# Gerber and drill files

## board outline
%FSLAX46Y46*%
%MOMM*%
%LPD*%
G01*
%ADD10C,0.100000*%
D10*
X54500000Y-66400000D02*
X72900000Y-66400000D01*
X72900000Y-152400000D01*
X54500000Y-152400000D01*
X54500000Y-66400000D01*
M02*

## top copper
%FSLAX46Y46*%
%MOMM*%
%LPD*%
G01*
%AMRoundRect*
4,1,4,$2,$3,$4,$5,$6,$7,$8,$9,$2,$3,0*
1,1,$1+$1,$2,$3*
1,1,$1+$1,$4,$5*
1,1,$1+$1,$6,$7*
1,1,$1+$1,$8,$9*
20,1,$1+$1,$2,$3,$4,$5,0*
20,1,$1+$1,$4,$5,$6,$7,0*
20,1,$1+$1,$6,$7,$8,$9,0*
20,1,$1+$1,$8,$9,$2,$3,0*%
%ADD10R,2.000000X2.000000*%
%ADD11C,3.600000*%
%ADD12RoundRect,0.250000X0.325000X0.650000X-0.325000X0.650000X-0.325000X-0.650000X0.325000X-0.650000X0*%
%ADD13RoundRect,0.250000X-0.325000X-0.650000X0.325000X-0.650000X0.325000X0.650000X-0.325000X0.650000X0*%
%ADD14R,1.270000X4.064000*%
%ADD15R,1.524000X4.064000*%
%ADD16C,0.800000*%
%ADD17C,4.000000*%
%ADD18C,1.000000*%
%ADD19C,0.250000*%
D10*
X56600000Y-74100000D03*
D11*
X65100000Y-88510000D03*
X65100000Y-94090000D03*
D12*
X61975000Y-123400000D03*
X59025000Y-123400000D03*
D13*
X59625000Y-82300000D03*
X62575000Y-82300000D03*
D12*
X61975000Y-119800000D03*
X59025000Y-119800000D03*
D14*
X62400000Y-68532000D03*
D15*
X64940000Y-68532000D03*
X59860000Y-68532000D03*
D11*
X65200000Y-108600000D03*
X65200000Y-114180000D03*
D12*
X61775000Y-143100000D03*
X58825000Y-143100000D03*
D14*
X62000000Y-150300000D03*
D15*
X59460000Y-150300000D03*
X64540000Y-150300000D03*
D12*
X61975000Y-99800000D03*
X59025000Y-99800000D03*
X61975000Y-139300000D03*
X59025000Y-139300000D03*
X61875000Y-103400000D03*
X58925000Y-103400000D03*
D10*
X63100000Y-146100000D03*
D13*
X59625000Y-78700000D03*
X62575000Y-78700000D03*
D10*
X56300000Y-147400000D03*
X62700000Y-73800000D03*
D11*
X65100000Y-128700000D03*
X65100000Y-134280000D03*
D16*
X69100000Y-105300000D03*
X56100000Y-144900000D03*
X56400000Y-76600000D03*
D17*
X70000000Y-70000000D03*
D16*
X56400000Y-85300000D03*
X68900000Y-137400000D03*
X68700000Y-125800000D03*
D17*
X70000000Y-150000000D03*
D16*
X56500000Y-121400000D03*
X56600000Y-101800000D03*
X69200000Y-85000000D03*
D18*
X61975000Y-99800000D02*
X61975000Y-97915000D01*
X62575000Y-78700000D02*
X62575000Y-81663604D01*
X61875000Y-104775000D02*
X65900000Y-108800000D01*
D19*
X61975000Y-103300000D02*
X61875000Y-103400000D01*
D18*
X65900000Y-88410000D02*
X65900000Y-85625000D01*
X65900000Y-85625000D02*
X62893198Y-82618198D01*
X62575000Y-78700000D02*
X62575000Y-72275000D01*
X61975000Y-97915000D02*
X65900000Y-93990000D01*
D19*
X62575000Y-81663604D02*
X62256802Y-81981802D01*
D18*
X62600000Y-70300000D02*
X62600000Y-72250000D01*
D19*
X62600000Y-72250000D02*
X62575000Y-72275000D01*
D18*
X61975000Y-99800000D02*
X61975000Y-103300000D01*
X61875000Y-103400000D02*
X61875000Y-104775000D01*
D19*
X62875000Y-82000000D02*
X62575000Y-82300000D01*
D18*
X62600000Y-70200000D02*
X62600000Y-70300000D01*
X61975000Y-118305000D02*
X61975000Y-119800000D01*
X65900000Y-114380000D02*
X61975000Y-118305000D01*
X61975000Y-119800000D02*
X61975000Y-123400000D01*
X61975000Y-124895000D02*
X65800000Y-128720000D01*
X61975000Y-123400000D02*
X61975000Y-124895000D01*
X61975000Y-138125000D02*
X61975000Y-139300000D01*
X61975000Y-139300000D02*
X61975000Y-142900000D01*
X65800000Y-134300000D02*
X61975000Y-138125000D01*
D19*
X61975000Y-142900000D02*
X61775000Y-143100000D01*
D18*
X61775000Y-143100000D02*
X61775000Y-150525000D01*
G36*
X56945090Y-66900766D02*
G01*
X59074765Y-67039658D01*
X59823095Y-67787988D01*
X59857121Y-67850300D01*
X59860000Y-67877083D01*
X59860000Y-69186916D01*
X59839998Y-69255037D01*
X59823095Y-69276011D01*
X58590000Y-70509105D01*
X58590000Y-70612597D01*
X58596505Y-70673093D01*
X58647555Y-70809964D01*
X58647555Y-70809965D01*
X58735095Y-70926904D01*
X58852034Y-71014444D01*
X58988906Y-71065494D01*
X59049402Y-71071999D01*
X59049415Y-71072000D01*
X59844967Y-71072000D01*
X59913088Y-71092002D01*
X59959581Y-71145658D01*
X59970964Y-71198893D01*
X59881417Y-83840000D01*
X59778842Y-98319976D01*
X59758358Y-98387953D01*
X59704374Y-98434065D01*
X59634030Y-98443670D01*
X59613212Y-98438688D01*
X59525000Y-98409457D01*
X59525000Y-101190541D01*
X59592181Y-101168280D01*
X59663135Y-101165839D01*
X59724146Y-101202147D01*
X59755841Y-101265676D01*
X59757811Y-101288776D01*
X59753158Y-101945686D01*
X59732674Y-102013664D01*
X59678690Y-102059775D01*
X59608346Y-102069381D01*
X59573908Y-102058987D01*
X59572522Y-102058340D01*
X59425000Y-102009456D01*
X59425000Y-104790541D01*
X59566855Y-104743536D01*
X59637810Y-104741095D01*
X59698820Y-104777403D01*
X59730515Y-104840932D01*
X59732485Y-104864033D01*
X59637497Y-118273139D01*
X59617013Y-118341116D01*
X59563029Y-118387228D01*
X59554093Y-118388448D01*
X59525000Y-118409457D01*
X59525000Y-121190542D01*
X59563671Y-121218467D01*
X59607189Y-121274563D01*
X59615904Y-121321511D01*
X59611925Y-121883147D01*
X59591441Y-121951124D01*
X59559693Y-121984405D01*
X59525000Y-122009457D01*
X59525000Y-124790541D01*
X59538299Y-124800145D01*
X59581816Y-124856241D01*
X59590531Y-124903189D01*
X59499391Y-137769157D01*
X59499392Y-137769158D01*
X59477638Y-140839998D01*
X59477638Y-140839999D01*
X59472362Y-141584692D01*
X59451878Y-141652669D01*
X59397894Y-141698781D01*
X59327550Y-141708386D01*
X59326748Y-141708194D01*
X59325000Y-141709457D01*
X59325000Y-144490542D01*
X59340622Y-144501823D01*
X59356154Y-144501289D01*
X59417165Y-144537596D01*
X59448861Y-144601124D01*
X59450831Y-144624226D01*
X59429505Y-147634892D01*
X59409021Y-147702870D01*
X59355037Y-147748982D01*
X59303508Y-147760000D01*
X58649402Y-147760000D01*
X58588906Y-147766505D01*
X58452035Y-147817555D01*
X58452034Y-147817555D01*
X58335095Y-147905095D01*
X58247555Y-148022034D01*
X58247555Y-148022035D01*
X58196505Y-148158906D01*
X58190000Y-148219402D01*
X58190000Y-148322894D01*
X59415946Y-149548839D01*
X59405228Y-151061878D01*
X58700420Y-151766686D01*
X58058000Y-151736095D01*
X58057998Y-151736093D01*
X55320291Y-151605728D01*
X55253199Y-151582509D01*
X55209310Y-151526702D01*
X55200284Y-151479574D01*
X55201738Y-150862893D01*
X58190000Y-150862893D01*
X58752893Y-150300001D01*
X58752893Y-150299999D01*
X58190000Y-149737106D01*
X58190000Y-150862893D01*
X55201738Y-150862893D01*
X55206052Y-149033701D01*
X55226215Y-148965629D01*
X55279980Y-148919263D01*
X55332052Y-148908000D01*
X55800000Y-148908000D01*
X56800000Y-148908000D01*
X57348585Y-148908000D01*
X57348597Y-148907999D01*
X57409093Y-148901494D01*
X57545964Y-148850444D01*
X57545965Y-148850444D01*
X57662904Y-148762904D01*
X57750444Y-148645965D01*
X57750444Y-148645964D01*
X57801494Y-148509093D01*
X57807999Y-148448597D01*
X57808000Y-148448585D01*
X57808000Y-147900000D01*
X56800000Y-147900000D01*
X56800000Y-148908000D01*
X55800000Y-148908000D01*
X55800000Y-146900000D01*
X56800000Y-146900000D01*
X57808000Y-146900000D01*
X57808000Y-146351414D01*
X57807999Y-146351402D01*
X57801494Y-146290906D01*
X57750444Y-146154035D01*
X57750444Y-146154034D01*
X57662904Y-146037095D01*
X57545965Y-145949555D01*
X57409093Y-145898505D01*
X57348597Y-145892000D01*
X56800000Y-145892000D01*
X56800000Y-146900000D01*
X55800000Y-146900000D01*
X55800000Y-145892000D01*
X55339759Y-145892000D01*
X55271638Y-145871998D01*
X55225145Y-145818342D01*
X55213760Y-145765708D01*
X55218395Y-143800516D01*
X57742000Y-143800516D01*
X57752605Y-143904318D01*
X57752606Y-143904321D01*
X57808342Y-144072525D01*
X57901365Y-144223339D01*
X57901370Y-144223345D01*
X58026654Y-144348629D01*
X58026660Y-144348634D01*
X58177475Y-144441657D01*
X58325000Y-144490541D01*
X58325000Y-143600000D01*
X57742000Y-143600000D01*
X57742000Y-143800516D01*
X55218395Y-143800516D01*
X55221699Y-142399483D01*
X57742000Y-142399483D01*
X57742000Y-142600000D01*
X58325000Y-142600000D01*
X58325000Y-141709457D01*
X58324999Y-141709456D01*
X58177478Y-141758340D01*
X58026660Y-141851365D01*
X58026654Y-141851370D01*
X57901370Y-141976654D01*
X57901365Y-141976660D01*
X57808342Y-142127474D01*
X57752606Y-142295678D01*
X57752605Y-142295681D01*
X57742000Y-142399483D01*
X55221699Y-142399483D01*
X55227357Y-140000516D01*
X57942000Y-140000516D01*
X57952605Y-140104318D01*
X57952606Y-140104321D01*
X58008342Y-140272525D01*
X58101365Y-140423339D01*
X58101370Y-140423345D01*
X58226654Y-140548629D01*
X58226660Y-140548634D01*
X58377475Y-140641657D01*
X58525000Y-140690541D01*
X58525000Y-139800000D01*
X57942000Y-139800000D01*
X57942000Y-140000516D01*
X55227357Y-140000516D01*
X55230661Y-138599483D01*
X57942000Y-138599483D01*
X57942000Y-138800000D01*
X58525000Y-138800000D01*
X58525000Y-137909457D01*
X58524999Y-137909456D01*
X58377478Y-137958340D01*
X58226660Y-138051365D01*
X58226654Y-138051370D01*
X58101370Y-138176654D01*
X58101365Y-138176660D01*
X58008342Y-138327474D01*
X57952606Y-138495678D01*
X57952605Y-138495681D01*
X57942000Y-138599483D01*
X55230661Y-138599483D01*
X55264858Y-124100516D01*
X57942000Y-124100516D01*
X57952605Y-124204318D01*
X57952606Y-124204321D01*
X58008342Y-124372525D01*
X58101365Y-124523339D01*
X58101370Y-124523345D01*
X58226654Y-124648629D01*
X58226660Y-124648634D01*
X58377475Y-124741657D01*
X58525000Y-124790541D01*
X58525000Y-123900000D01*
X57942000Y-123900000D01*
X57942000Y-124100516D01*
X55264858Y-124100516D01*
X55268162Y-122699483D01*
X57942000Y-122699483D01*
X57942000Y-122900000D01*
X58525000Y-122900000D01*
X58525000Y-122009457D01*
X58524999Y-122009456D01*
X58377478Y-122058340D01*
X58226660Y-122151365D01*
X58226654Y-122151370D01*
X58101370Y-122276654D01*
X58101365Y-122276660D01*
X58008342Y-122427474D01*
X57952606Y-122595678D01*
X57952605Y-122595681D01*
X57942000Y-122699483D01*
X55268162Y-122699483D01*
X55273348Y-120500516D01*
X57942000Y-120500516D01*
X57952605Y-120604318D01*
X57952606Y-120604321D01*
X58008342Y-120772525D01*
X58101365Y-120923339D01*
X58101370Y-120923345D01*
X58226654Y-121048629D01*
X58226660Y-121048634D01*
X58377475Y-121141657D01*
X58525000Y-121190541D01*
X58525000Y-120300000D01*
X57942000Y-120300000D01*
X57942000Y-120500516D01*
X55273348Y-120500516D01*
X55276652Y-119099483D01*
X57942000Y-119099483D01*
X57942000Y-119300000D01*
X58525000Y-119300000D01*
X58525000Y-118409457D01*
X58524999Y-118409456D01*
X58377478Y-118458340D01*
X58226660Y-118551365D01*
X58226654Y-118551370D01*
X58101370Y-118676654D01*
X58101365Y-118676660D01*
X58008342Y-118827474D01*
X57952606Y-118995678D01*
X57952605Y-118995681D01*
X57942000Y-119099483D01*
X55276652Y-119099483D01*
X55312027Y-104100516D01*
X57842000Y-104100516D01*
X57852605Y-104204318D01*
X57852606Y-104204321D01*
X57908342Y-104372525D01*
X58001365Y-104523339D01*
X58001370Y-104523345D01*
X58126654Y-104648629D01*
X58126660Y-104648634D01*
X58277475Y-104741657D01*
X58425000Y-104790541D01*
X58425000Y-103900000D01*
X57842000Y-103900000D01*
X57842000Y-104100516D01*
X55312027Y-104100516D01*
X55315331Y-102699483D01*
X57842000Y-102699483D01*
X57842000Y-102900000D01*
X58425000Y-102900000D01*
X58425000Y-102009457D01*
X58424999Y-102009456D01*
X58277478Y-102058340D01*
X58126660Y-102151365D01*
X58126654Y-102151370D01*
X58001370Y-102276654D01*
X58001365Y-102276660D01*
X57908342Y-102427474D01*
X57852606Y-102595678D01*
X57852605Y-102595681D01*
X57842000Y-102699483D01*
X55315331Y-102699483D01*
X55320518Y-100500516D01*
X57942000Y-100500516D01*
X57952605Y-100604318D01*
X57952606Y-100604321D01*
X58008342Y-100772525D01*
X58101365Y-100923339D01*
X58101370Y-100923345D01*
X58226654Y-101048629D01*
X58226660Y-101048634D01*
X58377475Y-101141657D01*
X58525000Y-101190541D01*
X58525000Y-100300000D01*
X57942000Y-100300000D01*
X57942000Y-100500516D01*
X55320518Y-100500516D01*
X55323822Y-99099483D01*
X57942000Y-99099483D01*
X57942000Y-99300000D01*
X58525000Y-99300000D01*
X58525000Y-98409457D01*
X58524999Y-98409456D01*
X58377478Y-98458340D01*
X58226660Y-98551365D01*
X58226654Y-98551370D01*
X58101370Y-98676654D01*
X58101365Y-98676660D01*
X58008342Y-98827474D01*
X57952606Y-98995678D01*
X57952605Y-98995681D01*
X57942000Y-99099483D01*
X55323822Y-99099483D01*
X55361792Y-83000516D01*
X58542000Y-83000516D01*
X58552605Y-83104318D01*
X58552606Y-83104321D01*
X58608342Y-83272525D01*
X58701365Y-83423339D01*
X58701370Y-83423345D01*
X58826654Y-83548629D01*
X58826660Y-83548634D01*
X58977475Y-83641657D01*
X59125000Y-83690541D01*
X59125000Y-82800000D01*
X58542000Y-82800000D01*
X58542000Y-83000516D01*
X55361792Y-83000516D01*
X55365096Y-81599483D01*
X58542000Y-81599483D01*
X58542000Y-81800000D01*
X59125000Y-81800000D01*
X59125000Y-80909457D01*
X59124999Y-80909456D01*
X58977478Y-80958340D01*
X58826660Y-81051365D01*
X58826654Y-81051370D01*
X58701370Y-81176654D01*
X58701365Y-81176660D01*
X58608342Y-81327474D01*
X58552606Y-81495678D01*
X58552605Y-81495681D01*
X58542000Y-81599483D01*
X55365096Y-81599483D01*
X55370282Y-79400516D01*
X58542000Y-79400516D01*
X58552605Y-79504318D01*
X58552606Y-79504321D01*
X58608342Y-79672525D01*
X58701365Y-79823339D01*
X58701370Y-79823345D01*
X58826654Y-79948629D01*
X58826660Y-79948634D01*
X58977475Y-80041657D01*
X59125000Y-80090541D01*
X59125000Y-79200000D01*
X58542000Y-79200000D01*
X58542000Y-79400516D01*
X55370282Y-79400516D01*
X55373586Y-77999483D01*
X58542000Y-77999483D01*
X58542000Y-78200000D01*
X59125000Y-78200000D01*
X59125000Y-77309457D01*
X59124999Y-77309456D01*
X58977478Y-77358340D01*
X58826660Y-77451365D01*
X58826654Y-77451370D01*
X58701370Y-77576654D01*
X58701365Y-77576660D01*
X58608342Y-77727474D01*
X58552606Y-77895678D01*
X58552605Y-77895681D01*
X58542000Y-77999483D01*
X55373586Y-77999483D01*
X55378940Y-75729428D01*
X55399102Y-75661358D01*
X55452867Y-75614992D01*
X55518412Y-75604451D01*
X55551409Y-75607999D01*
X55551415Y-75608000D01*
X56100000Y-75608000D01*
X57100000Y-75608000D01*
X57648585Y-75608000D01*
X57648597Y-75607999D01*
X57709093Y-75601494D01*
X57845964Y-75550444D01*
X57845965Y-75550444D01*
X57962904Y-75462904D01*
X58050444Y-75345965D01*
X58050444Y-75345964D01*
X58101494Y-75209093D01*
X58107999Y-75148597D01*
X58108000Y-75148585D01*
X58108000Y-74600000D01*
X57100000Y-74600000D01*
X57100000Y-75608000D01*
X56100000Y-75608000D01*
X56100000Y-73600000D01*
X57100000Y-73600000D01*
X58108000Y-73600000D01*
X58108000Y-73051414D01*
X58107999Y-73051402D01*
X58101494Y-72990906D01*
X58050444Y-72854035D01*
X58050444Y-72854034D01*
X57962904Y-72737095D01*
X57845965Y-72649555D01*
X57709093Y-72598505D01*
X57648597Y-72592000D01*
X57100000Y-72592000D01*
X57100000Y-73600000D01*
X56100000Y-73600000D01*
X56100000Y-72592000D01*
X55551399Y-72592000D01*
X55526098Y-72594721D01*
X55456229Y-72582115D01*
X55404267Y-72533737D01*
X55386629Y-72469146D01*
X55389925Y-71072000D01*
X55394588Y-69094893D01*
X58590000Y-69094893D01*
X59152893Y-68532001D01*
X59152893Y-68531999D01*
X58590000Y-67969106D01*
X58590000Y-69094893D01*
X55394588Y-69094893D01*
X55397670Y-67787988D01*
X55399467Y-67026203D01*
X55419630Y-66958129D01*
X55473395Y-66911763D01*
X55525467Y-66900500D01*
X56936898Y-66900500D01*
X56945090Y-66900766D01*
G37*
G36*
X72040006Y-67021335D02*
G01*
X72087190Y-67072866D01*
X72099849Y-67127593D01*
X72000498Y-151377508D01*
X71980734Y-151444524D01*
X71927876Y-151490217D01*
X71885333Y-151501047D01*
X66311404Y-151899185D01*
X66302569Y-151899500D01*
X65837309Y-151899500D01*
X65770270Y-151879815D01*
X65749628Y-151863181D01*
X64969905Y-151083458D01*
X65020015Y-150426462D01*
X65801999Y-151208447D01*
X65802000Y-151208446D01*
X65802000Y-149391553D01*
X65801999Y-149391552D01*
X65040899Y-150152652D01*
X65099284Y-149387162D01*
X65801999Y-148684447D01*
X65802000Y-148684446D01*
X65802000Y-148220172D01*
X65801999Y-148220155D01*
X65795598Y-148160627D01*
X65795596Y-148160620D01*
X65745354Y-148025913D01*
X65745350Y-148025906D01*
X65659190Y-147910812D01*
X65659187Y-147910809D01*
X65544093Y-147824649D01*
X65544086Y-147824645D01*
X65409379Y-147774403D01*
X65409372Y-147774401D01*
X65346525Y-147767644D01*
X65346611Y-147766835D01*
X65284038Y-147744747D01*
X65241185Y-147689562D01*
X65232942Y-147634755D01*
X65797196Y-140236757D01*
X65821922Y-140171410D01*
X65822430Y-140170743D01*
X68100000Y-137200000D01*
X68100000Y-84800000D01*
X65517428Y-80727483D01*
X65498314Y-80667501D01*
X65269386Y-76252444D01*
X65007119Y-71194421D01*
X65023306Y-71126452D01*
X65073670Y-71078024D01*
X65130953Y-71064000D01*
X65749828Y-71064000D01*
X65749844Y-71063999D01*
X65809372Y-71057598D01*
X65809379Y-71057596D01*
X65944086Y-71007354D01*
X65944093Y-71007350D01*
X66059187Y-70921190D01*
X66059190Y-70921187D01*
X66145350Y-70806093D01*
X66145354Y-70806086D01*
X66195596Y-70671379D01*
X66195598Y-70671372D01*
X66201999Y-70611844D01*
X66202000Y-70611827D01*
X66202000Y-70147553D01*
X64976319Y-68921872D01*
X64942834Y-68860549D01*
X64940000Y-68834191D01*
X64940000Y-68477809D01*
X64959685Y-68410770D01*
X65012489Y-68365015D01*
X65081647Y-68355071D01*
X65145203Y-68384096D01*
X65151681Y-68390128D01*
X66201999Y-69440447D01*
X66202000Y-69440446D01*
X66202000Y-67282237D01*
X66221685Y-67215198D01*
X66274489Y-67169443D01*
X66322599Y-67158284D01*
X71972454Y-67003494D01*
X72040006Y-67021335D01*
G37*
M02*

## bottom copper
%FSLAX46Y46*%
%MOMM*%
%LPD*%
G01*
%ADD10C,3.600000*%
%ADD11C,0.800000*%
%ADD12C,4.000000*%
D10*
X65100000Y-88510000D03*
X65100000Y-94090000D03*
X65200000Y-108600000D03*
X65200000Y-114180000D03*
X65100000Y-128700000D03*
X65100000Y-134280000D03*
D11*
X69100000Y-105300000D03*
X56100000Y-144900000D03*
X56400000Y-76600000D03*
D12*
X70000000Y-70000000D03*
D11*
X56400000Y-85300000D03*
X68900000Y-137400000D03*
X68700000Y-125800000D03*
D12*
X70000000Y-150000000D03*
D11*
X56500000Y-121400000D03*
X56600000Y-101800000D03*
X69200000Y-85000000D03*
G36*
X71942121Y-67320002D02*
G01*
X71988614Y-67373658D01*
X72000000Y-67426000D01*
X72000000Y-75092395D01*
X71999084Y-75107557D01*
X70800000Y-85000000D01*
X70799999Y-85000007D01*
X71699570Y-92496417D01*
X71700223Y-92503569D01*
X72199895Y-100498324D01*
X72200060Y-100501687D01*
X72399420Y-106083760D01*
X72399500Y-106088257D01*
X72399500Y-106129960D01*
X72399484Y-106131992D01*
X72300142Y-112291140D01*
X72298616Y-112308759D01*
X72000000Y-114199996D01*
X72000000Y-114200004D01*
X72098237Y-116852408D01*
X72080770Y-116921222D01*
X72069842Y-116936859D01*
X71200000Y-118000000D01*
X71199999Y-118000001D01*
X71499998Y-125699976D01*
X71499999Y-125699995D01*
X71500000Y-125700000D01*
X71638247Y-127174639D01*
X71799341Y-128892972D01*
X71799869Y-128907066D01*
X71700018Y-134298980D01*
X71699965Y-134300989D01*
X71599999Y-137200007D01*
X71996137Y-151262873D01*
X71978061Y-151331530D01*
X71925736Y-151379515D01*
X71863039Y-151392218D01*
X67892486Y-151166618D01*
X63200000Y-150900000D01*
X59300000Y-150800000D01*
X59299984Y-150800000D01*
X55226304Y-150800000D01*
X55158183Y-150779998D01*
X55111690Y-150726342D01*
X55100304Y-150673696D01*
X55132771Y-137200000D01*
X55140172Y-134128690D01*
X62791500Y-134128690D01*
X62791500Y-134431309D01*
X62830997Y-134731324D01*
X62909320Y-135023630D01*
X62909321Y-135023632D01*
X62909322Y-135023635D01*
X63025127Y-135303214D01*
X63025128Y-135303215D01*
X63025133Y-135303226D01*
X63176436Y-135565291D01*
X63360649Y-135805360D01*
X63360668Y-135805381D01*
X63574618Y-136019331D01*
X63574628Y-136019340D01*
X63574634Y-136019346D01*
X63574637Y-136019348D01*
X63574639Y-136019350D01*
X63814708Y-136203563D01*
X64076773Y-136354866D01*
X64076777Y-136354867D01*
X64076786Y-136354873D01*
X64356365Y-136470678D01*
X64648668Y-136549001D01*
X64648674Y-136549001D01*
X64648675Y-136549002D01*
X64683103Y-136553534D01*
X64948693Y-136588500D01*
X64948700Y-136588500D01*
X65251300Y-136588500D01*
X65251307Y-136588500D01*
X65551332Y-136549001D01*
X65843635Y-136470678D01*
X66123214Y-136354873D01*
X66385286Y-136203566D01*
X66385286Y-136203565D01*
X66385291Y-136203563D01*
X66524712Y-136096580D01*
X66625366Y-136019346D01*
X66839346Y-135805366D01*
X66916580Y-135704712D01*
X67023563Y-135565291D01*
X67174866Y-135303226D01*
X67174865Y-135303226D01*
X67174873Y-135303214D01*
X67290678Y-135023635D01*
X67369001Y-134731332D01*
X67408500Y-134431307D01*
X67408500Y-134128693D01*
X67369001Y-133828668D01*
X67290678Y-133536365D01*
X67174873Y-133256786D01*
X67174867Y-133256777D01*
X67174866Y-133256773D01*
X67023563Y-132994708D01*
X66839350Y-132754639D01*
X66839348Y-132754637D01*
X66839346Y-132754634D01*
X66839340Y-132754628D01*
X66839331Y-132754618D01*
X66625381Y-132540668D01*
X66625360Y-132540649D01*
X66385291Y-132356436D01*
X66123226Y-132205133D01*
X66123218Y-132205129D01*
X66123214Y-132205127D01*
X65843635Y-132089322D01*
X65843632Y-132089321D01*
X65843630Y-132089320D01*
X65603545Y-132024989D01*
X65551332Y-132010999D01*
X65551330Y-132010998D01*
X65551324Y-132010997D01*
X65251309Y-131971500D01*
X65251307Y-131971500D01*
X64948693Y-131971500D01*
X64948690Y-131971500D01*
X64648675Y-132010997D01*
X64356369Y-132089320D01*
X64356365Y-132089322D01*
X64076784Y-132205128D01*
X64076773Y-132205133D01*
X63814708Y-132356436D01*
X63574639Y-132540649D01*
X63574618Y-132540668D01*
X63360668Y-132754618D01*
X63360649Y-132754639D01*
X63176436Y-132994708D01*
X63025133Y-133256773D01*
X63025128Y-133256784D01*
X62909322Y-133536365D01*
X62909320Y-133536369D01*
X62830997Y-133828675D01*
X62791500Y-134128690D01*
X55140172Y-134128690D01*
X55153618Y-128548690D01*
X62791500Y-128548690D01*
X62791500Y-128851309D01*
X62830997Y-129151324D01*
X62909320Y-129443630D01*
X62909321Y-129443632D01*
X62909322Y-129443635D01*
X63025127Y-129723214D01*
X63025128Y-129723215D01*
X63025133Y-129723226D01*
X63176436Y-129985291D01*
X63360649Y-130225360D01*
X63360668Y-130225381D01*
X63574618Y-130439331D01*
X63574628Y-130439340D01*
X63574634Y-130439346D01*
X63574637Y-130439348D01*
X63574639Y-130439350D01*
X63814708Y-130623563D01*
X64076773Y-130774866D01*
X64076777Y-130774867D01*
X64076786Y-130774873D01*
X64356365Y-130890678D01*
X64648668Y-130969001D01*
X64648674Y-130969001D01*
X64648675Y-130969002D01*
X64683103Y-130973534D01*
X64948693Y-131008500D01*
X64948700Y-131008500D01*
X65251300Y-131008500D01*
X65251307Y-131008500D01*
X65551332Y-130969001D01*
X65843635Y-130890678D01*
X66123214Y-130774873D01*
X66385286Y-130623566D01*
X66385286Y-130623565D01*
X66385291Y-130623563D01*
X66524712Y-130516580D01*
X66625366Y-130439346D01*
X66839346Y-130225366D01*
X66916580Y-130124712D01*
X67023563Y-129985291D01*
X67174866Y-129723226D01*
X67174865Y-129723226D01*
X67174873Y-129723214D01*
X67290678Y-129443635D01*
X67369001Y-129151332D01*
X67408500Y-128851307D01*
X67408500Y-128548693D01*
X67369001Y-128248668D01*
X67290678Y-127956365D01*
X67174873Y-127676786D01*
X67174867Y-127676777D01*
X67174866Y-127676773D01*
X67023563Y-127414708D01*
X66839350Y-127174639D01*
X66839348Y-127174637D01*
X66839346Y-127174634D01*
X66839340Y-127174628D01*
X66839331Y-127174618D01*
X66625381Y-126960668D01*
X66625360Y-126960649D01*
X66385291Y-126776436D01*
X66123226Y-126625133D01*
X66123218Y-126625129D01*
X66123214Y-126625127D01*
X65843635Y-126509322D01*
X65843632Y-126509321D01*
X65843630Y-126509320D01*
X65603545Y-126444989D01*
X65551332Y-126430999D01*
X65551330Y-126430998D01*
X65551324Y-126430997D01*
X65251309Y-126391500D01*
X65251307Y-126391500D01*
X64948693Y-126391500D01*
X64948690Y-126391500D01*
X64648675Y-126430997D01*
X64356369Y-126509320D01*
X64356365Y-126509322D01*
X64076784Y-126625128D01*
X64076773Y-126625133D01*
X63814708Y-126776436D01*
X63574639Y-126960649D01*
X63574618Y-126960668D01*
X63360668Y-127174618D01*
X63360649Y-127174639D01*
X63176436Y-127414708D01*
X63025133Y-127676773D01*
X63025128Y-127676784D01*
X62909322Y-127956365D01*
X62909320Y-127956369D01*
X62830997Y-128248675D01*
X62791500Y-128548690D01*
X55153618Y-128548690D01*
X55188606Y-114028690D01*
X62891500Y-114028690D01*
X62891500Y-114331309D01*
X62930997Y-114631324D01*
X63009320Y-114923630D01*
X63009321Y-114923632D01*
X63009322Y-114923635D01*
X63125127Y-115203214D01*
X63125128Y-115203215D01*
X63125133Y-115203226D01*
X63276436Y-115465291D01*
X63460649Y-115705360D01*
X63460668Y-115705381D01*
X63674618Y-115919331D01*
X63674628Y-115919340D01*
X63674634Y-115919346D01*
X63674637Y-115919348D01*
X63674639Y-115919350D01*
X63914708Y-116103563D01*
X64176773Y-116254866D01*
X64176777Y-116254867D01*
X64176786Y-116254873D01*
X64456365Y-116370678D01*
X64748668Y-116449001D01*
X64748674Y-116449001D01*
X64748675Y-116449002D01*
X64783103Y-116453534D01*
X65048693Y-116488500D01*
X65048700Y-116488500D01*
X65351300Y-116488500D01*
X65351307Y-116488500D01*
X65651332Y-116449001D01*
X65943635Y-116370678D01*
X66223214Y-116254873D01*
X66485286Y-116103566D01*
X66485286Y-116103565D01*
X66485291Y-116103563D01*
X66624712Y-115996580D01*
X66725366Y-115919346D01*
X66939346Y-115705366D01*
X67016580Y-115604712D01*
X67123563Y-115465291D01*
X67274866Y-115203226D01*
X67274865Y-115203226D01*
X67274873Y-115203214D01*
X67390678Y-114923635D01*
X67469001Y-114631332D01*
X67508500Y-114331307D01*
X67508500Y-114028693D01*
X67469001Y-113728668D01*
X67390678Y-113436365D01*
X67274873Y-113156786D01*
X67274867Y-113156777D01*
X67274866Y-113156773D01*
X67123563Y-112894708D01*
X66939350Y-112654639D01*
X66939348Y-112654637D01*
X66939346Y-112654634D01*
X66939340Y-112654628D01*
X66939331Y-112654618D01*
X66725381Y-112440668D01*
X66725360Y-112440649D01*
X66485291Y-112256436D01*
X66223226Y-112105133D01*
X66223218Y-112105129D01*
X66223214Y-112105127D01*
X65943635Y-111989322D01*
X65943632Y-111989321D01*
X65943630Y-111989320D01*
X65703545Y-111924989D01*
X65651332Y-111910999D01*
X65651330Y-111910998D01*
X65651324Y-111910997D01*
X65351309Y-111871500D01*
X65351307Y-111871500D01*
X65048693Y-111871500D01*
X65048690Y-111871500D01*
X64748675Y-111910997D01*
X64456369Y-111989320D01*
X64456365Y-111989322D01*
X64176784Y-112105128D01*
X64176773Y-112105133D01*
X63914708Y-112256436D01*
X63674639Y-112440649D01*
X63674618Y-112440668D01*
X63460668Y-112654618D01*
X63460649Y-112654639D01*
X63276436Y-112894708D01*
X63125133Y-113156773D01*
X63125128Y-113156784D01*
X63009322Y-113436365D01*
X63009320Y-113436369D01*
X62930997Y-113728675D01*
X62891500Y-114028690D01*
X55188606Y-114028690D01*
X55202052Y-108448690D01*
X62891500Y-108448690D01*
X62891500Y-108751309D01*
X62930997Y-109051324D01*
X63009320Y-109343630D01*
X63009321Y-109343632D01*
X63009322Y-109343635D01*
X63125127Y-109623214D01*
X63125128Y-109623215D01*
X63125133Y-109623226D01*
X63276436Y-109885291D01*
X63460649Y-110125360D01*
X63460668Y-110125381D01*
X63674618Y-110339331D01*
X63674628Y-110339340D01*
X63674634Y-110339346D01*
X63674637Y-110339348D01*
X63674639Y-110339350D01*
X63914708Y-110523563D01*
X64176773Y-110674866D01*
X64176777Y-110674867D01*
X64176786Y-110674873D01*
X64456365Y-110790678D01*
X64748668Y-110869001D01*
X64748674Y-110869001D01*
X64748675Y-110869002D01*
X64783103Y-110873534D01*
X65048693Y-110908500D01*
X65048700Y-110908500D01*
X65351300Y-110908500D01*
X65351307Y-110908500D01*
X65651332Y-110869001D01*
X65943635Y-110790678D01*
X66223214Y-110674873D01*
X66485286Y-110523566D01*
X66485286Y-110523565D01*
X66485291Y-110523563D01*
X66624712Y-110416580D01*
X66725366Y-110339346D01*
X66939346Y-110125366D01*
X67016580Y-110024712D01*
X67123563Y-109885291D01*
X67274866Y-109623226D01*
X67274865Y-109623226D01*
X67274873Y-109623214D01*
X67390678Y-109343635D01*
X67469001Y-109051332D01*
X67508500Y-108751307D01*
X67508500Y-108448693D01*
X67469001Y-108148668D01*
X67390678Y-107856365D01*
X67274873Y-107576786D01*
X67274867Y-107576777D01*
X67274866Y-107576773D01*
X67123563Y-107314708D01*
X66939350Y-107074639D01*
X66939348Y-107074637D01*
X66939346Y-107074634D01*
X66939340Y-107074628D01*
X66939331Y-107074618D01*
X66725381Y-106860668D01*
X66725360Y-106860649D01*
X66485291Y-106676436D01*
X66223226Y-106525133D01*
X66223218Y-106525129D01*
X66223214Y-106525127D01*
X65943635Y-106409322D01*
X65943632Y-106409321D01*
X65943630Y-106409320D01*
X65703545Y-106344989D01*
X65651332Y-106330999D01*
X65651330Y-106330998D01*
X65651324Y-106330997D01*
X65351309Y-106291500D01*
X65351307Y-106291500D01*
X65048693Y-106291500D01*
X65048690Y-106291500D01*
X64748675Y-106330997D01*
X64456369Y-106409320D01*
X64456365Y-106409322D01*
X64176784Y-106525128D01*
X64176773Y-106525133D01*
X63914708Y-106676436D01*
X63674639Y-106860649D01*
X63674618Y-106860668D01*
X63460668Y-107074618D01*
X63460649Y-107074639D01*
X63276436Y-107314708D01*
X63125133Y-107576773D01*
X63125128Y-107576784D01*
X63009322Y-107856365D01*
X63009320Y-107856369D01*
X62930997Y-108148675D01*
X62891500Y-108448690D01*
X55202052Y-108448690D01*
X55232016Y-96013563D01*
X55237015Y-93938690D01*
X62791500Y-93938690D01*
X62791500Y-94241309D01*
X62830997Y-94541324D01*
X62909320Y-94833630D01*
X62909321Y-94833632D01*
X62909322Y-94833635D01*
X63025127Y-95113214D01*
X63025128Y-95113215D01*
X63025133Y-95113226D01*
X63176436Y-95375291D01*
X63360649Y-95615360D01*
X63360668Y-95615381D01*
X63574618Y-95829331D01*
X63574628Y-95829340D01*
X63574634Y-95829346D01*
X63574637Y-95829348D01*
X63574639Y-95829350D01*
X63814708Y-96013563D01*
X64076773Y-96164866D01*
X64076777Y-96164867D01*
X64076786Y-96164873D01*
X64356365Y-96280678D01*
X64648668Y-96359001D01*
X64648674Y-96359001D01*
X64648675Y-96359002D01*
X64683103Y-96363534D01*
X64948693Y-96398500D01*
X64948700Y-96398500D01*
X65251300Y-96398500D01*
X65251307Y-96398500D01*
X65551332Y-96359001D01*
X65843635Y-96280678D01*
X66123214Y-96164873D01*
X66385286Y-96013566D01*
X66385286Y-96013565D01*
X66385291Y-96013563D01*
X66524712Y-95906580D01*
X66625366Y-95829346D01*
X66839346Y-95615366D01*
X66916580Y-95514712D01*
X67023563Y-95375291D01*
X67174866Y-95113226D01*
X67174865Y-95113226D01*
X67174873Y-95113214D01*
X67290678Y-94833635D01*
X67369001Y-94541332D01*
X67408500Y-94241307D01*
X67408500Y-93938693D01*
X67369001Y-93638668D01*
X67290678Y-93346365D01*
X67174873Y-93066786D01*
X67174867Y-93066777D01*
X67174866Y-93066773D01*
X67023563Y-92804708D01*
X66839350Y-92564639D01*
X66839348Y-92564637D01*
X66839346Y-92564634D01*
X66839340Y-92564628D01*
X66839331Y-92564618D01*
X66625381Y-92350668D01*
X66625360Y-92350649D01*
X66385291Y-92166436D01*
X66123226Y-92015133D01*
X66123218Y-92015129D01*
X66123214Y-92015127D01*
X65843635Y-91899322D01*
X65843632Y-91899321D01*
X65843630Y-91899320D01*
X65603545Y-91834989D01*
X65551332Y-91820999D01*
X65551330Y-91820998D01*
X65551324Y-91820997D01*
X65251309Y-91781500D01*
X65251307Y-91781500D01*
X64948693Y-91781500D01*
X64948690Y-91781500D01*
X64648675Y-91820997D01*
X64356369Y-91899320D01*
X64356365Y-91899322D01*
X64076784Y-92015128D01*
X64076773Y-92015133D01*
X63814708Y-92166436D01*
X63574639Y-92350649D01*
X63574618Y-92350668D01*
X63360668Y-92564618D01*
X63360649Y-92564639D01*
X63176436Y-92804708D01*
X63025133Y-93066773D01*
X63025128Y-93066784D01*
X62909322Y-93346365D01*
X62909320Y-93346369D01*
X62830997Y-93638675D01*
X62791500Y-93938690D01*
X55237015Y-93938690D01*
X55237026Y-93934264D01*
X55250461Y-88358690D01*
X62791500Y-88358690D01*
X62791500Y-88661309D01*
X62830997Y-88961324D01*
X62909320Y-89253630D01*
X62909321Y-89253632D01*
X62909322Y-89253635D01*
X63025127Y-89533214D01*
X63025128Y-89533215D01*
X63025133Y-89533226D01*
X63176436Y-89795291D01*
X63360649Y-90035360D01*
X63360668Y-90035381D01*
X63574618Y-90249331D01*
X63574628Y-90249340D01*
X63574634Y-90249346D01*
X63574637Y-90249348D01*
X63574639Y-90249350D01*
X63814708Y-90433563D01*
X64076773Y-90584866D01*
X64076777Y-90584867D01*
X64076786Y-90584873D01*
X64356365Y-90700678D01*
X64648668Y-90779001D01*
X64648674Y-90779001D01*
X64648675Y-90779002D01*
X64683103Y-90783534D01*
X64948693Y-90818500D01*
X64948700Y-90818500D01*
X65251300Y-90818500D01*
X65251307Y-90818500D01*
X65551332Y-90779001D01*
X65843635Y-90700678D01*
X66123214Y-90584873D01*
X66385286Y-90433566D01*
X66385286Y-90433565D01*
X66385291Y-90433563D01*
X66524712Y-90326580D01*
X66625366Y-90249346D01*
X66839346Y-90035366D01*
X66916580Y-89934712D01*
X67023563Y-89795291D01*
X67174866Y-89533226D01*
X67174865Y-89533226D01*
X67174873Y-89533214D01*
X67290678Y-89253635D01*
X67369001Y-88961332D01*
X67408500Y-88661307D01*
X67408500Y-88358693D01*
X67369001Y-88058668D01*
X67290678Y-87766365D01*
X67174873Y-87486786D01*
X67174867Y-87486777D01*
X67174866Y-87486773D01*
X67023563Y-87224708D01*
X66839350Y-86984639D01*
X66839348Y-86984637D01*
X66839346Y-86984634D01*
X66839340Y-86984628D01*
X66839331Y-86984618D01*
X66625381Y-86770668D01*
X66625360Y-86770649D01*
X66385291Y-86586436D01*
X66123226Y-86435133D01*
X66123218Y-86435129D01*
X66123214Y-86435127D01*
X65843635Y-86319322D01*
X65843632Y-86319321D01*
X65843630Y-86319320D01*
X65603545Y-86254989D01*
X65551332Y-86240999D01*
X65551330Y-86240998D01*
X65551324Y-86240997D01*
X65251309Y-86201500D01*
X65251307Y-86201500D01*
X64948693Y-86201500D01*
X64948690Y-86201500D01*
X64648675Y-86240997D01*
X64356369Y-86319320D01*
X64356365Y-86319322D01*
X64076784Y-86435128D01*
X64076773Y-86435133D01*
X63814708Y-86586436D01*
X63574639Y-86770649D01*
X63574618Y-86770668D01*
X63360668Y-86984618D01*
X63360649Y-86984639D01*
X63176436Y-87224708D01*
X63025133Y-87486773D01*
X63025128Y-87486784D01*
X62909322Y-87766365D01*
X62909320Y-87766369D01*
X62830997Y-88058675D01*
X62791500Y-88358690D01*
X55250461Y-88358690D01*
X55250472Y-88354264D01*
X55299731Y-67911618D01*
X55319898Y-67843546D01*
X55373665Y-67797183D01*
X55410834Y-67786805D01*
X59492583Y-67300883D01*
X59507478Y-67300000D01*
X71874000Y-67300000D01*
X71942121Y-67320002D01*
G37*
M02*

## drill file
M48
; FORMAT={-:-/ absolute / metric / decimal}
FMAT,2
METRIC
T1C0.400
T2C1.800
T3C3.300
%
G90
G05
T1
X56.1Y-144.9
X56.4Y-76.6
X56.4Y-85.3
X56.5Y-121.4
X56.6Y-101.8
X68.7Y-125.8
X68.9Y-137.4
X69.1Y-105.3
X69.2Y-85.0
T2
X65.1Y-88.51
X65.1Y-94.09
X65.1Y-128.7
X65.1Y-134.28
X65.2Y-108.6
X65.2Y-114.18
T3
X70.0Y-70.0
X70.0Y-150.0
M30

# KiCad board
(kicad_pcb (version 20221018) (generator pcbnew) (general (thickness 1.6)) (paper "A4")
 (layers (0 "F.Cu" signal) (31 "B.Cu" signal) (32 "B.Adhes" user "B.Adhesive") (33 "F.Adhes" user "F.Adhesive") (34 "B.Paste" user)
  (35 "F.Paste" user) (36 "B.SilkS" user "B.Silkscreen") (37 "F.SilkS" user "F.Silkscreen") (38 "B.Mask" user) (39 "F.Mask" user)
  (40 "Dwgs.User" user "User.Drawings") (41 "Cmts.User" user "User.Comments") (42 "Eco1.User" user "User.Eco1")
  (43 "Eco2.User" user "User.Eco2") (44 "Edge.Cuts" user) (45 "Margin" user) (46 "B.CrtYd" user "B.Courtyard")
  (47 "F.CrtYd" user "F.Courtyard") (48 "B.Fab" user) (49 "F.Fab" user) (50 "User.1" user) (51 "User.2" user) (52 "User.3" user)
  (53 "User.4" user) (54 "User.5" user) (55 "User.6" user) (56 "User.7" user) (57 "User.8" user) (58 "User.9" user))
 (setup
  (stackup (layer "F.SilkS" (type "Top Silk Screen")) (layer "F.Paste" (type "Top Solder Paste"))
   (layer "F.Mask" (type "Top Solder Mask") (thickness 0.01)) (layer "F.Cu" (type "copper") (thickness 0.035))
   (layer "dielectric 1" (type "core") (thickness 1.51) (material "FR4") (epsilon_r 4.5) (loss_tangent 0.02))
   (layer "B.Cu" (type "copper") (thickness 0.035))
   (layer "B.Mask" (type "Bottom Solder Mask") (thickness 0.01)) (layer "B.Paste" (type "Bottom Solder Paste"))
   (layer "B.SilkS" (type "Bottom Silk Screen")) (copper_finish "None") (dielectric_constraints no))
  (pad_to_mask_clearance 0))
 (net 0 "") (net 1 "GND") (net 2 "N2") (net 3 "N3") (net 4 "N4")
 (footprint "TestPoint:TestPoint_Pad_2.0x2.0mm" (layer "F.Cu") (at 56.6 74.1)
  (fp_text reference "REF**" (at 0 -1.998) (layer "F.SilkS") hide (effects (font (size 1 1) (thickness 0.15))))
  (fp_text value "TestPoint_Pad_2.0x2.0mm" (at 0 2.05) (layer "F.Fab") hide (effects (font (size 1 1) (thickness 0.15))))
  (pad "1" smd rect (at 0 0) (size 2 2) (layers "F.Cu" "F.Mask") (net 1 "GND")))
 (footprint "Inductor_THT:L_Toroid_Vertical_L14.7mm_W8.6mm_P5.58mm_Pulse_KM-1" (layer "F.Cu") (at 65.1 88.51)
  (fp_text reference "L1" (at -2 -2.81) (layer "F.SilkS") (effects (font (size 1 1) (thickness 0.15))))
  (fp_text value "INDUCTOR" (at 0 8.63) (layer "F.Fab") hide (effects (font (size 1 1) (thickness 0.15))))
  (pad "1" thru_hole circle (at 0 0) (size 3.6 3.6) (drill 1.8) (layers "*.Cu" "*.Mask") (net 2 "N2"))
  (pad "2" thru_hole circle (at 0 5.58) (size 3.6 3.6) (drill 1.8) (layers "*.Cu" "*.Mask") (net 2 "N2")))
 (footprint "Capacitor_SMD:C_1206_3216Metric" (layer "F.Cu") (at 60.5 123.4 180)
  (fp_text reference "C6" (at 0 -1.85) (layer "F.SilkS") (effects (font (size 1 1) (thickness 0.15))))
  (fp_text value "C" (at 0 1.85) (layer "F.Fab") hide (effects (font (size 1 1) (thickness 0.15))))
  (pad "1" smd roundrect (at -1.475 0 180) (size 1.15 1.8) (layers "F.Cu" "F.Paste" "F.Mask") (roundrect_rratio 0.2173913043) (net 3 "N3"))
  (pad "2" smd roundrect (at 1.475 0 180) (size 1.15 1.8) (layers "F.Cu" "F.Paste" "F.Mask") (roundrect_rratio 0.2173913043) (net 1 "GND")))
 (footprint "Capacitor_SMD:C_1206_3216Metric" (layer "F.Cu") (at 61.1 82.3)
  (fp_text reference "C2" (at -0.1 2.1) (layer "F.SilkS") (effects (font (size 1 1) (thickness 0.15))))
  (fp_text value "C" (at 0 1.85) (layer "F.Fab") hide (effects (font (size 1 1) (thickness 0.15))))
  (pad "1" smd roundrect (at -1.475 0) (size 1.15 1.8) (layers "F.Cu" "F.Paste" "F.Mask") (roundrect_rratio 0.2173913043) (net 1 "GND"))
  (pad "2" smd roundrect (at 1.475 0) (size 1.15 1.8) (layers "F.Cu" "F.Paste" "F.Mask") (roundrect_rratio 0.2173913043) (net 2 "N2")))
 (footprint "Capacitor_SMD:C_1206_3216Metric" (layer "F.Cu") (at 60.5 119.8 180)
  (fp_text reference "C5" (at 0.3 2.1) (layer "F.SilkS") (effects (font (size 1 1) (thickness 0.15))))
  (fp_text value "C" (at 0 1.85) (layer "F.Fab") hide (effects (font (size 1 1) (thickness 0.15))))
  (pad "1" smd roundrect (at -1.475 0 180) (size 1.15 1.8) (layers "F.Cu" "F.Paste" "F.Mask") (roundrect_rratio 0.2173913043) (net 3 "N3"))
  (pad "2" smd roundrect (at 1.475 0 180) (size 1.15 1.8) (layers "F.Cu" "F.Paste" "F.Mask") (roundrect_rratio 0.2173913043) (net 1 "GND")))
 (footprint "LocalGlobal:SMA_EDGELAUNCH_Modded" (layer "F.Cu") (at 62.4 66.5 -90)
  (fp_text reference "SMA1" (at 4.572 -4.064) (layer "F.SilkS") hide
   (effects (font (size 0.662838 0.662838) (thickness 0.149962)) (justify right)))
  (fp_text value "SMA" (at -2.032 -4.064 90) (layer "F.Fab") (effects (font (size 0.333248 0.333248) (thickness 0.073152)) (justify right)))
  (pad "1" smd rect (at 2.032 0) (size 1.27 4.064) (layers "F.Cu" "F.Mask") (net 2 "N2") (solder_mask_margin 0.0508) (zone_connect 2)
   (thermal_bridge_angle 45))
  (pad "2" smd rect (at 2.032 -2.54) (size 1.524 4.064) (layers "F.Cu" "F.Mask") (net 1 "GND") (solder_mask_margin 0.0508)
   (thermal_bridge_angle 45))
  (pad "2" smd rect (at 2.032 2.54) (size 1.524 4.064) (layers "F.Cu" "F.Mask") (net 1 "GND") (solder_mask_margin 0.0508)
   (thermal_bridge_angle 45)))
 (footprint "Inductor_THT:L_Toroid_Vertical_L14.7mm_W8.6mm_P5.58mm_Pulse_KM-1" (layer "F.Cu") (at 65.2 108.6)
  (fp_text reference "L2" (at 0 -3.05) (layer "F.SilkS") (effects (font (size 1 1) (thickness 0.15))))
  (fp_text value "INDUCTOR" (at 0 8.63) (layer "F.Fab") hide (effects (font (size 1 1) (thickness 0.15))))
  (pad "1" thru_hole circle (at 0 0) (size 3.6 3.6) (drill 1.8) (layers "*.Cu" "*.Mask") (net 2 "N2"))
  (pad "2" thru_hole circle (at 0 5.58) (size 3.6 3.6) (drill 1.8) (layers "*.Cu" "*.Mask") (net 3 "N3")))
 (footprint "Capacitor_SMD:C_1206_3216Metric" (layer "F.Cu") (at 60.3 143.1 180)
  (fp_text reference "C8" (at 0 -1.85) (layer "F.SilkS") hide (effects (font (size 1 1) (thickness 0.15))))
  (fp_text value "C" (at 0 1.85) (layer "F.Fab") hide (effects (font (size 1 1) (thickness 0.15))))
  (pad "1" smd roundrect (at -1.475 0 180) (size 1.15 1.8) (layers "F.Cu" "F.Paste" "F.Mask") (roundrect_rratio 0.2173913043) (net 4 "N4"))
  (pad "2" smd roundrect (at 1.475 0 180) (size 1.15 1.8) (layers "F.Cu" "F.Paste" "F.Mask") (roundrect_rratio 0.2173913043) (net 1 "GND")))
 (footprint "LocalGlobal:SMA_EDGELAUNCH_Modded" (layer "F.Cu") (at 62 152.332 90)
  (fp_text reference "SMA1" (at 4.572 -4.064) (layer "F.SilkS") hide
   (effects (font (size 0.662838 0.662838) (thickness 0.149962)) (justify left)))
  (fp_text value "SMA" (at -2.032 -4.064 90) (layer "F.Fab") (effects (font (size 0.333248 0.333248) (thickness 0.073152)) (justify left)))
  (pad "1" smd rect (at 2.032 0 180) (size 1.27 4.064) (layers "F.Cu" "F.Mask") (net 4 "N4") (solder_mask_margin 0.0508) (zone_connect 2)
   (thermal_bridge_angle 45))
  (pad "2" smd rect (at 2.032 -2.54 180) (size 1.524 4.064) (layers "F.Cu" "F.Mask") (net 1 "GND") (solder_mask_margin 0.0508)
   (thermal_bridge_angle 45))
  (pad "2" smd rect (at 2.032 2.54 180) (size 1.524 4.064) (layers "F.Cu" "F.Mask") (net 1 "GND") (solder_mask_margin 0.0508)
   (thermal_bridge_angle 45)))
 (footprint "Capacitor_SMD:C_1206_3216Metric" (layer "F.Cu") (at 60.5 99.8 180)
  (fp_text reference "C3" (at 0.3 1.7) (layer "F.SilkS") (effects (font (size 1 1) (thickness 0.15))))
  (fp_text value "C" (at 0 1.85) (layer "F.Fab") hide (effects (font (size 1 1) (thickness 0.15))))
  (pad "1" smd roundrect (at -1.475 0 180) (size 1.15 1.8) (layers "F.Cu" "F.Paste" "F.Mask") (roundrect_rratio 0.2173913043) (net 2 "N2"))
  (pad "2" smd roundrect (at 1.475 0 180) (size 1.15 1.8) (layers "F.Cu" "F.Paste" "F.Mask") (roundrect_rratio 0.2173913043) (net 1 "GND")))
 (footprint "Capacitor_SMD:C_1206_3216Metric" (layer "F.Cu") (at 60.5 139.3 180)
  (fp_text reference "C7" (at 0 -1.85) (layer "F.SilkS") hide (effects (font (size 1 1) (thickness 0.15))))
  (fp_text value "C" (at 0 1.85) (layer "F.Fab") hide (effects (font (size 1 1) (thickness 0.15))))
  (pad "1" smd roundrect (at -1.475 0 180) (size 1.15 1.8) (layers "F.Cu" "F.Paste" "F.Mask") (roundrect_rratio 0.2173913043) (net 4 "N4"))
  (pad "2" smd roundrect (at 1.475 0 180) (size 1.15 1.8) (layers "F.Cu" "F.Paste" "F.Mask") (roundrect_rratio 0.2173913043) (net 1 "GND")))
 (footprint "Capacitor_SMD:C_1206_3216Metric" (layer "F.Cu") (at 60.4 103.4 180)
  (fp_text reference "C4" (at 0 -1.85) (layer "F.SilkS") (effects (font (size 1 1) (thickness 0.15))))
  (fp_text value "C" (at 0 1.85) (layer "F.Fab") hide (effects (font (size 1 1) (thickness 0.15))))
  (pad "1" smd roundrect (at -1.475 0 180) (size 1.15 1.8) (layers "F.Cu" "F.Paste" "F.Mask") (roundrect_rratio 0.2173913043) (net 2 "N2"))
  (pad "2" smd roundrect (at 1.475 0 180) (size 1.15 1.8) (layers "F.Cu" "F.Paste" "F.Mask") (roundrect_rratio 0.2173913043) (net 1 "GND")))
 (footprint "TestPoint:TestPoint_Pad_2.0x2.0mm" (layer "F.Cu") (at 63.1 146.1)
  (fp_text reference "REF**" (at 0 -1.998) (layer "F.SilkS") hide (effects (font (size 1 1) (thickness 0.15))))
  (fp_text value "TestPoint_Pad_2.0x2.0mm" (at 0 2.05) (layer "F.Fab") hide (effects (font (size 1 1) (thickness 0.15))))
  (pad "1" smd rect (at 0 0) (size 2 2) (layers "F.Cu" "F.Mask") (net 4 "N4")))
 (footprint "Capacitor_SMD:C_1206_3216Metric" (layer "F.Cu") (at 61.1 78.7)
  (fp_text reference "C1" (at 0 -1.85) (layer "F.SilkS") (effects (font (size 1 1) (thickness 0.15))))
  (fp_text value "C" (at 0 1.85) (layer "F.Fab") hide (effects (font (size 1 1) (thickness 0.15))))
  (pad "1" smd roundrect (at -1.475 0) (size 1.15 1.8) (layers "F.Cu" "F.Paste" "F.Mask") (roundrect_rratio 0.2173913043) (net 1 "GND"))
  (pad "2" smd roundrect (at 1.475 0) (size 1.15 1.8) (layers "F.Cu" "F.Paste" "F.Mask") (roundrect_rratio 0.2173913043) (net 2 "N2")))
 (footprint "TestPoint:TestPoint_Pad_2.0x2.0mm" (layer "F.Cu") (at 56.3 147.4)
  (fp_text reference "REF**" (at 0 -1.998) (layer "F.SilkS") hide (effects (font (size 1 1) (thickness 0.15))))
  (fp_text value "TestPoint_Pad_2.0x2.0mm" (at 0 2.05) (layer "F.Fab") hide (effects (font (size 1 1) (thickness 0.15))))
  (pad "1" smd rect (at 0 0) (size 2 2) (layers "F.Cu" "F.Mask") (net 1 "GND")))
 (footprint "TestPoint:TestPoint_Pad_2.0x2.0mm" (layer "F.Cu") (at 62.7 73.8)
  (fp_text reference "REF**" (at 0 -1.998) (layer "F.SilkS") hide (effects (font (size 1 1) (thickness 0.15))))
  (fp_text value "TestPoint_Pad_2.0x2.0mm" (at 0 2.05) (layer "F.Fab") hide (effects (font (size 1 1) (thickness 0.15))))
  (pad "1" smd rect (at 0 0) (size 2 2) (layers "F.Cu" "F.Mask") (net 2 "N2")))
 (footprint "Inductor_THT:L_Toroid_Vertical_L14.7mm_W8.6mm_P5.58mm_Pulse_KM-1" (layer "F.Cu") (at 65.1 128.7)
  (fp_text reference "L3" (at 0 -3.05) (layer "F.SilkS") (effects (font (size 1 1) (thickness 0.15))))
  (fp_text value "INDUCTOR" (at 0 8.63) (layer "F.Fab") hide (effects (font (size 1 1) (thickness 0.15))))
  (pad "1" thru_hole circle (at 0 0) (size 3.6 3.6) (drill 1.8) (layers "*.Cu" "*.Mask") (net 3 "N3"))
  (pad "2" thru_hole circle (at 0 5.58) (size 3.6 3.6) (drill 1.8) (layers "*.Cu" "*.Mask") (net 4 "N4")))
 (gr_rect (start 54.5 66.4) (end 72.9 152.4) (stroke (width 0.1) (type solid)) (fill none) (layer "Edge.Cuts"))
 (via (at 69.1 105.3) (size 0.8) (drill 0.4) (layers "F.Cu" "B.Cu") (free) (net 1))
 (via (at 56.1 144.9) (size 0.8) (drill 0.4) (layers "F.Cu" "B.Cu") (free) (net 1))
 (via (at 56.4 76.6) (size 0.8) (drill 0.4) (layers "F.Cu" "B.Cu") (free) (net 1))
 (via (at 70 70) (size 4) (drill 3.3) (layers "F.Cu" "B.Cu") (free) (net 1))
 (via (at 56.4 85.3) (size 0.8) (drill 0.4) (layers "F.Cu" "B.Cu") (free) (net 1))
 (via (at 68.9 137.4) (size 0.8) (drill 0.4) (layers "F.Cu" "B.Cu") (free) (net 1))
 (via (at 68.7 125.8) (size 0.8) (drill 0.4) (layers "F.Cu" "B.Cu") (free) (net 1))
 (via (at 70 150) (size 4) (drill 3.3) (layers "F.Cu" "B.Cu") (free) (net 1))
 (via (at 56.5 121.4) (size 0.8) (drill 0.4) (layers "F.Cu" "B.Cu") (free) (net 1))
 (via (at 56.6 101.8) (size 0.8) (drill 0.4) (layers "F.Cu" "B.Cu") (free) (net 1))
 (via (at 69.2 85) (size 0.8) (drill 0.4) (layers "F.Cu" "B.Cu") (free) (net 1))
 (segment (start 61.975 99.8) (end 61.975 97.915) (width 1) (layer "F.Cu") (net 2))
 (segment (start 62.575 78.7) (end 62.575 81.663604) (width 1) (layer "F.Cu") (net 2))
 (segment (start 61.875 104.775) (end 65.9 108.8) (width 1) (layer "F.Cu") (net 2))
 (segment (start 61.975 103.3) (end 61.875 103.4) (width 0.25) (layer "F.Cu") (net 2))
 (segment (start 65.9 88.41) (end 65.9 85.625) (width 1) (layer "F.Cu") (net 2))
 (segment (start 65.9 85.625) (end 62.893198 82.618198) (width 1) (layer "F.Cu") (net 2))
 (segment (start 62.575 78.7) (end 62.575 72.275) (width 1) (layer "F.Cu") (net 2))
 (segment (start 61.975 97.915) (end 65.9 93.99) (width 1) (layer "F.Cu") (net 2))
 (segment (start 62.575 81.663604) (end 62.256802 81.981802) (width 0.25) (layer "F.Cu") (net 2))
 (segment (start 62.6 70.3) (end 62.6 72.25) (width 1) (layer "F.Cu") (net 2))
 (segment (start 62.6 72.25) (end 62.575 72.275) (width 0.25) (layer "F.Cu") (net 2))
 (segment (start 61.975 99.8) (end 61.975 103.3) (width 1) (layer "F.Cu") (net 2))
 (segment (start 61.875 103.4) (end 61.875 104.775) (width 1) (layer "F.Cu") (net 2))
 (segment (start 62.875 82) (end 62.575 82.3) (width 0.25) (layer "F.Cu") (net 2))
 (segment (start 62.6 70.2) (end 62.6 70.3) (width 1) (layer "F.Cu") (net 2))
 (segment (start 61.975 118.305) (end 61.975 119.8) (width 1) (layer "F.Cu") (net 3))
 (segment (start 65.9 114.38) (end 61.975 118.305) (width 1) (layer "F.Cu") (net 3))
 (segment (start 61.975 119.8) (end 61.975 123.4) (width 1) (layer "F.Cu") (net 3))
 (segment (start 61.975 124.895) (end 65.8 128.72) (width 1) (layer "F.Cu") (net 3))
 (segment (start 61.975 123.4) (end 61.975 124.895) (width 1) (layer "F.Cu") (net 3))
 (segment (start 61.975 138.125) (end 61.975 139.3) (width 1) (layer "F.Cu") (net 4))
 (segment (start 61.975 139.3) (end 61.975 142.9) (width 1) (layer "F.Cu") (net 4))
 (segment (start 65.8 134.3) (end 61.975 138.125) (width 1) (layer "F.Cu") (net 4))
 (segment (start 61.975 142.9) (end 61.775 143.1) (width 0.25) (layer "F.Cu") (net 4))
 (segment (start 61.775 143.1) (end 61.775 150.525) (width 1) (layer "F.Cu") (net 4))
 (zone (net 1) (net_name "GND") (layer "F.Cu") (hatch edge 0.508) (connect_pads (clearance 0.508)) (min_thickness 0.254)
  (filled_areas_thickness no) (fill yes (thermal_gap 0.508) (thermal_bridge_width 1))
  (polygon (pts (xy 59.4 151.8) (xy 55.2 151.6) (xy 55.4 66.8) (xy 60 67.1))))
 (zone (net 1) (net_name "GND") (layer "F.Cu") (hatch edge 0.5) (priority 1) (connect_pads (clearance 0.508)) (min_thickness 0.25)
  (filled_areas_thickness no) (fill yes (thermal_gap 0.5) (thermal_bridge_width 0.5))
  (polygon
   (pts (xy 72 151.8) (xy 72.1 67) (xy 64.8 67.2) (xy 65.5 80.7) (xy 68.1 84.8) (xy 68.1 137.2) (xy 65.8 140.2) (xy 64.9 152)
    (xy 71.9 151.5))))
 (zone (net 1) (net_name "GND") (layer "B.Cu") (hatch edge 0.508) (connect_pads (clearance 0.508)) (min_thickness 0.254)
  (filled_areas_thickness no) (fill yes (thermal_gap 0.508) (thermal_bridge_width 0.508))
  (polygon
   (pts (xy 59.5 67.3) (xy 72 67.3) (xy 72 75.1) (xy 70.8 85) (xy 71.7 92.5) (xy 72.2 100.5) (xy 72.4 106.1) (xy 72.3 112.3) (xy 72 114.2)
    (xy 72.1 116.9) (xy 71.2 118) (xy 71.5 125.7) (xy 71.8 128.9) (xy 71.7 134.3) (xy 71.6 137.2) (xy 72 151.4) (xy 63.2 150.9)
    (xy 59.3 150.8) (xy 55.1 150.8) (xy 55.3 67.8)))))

